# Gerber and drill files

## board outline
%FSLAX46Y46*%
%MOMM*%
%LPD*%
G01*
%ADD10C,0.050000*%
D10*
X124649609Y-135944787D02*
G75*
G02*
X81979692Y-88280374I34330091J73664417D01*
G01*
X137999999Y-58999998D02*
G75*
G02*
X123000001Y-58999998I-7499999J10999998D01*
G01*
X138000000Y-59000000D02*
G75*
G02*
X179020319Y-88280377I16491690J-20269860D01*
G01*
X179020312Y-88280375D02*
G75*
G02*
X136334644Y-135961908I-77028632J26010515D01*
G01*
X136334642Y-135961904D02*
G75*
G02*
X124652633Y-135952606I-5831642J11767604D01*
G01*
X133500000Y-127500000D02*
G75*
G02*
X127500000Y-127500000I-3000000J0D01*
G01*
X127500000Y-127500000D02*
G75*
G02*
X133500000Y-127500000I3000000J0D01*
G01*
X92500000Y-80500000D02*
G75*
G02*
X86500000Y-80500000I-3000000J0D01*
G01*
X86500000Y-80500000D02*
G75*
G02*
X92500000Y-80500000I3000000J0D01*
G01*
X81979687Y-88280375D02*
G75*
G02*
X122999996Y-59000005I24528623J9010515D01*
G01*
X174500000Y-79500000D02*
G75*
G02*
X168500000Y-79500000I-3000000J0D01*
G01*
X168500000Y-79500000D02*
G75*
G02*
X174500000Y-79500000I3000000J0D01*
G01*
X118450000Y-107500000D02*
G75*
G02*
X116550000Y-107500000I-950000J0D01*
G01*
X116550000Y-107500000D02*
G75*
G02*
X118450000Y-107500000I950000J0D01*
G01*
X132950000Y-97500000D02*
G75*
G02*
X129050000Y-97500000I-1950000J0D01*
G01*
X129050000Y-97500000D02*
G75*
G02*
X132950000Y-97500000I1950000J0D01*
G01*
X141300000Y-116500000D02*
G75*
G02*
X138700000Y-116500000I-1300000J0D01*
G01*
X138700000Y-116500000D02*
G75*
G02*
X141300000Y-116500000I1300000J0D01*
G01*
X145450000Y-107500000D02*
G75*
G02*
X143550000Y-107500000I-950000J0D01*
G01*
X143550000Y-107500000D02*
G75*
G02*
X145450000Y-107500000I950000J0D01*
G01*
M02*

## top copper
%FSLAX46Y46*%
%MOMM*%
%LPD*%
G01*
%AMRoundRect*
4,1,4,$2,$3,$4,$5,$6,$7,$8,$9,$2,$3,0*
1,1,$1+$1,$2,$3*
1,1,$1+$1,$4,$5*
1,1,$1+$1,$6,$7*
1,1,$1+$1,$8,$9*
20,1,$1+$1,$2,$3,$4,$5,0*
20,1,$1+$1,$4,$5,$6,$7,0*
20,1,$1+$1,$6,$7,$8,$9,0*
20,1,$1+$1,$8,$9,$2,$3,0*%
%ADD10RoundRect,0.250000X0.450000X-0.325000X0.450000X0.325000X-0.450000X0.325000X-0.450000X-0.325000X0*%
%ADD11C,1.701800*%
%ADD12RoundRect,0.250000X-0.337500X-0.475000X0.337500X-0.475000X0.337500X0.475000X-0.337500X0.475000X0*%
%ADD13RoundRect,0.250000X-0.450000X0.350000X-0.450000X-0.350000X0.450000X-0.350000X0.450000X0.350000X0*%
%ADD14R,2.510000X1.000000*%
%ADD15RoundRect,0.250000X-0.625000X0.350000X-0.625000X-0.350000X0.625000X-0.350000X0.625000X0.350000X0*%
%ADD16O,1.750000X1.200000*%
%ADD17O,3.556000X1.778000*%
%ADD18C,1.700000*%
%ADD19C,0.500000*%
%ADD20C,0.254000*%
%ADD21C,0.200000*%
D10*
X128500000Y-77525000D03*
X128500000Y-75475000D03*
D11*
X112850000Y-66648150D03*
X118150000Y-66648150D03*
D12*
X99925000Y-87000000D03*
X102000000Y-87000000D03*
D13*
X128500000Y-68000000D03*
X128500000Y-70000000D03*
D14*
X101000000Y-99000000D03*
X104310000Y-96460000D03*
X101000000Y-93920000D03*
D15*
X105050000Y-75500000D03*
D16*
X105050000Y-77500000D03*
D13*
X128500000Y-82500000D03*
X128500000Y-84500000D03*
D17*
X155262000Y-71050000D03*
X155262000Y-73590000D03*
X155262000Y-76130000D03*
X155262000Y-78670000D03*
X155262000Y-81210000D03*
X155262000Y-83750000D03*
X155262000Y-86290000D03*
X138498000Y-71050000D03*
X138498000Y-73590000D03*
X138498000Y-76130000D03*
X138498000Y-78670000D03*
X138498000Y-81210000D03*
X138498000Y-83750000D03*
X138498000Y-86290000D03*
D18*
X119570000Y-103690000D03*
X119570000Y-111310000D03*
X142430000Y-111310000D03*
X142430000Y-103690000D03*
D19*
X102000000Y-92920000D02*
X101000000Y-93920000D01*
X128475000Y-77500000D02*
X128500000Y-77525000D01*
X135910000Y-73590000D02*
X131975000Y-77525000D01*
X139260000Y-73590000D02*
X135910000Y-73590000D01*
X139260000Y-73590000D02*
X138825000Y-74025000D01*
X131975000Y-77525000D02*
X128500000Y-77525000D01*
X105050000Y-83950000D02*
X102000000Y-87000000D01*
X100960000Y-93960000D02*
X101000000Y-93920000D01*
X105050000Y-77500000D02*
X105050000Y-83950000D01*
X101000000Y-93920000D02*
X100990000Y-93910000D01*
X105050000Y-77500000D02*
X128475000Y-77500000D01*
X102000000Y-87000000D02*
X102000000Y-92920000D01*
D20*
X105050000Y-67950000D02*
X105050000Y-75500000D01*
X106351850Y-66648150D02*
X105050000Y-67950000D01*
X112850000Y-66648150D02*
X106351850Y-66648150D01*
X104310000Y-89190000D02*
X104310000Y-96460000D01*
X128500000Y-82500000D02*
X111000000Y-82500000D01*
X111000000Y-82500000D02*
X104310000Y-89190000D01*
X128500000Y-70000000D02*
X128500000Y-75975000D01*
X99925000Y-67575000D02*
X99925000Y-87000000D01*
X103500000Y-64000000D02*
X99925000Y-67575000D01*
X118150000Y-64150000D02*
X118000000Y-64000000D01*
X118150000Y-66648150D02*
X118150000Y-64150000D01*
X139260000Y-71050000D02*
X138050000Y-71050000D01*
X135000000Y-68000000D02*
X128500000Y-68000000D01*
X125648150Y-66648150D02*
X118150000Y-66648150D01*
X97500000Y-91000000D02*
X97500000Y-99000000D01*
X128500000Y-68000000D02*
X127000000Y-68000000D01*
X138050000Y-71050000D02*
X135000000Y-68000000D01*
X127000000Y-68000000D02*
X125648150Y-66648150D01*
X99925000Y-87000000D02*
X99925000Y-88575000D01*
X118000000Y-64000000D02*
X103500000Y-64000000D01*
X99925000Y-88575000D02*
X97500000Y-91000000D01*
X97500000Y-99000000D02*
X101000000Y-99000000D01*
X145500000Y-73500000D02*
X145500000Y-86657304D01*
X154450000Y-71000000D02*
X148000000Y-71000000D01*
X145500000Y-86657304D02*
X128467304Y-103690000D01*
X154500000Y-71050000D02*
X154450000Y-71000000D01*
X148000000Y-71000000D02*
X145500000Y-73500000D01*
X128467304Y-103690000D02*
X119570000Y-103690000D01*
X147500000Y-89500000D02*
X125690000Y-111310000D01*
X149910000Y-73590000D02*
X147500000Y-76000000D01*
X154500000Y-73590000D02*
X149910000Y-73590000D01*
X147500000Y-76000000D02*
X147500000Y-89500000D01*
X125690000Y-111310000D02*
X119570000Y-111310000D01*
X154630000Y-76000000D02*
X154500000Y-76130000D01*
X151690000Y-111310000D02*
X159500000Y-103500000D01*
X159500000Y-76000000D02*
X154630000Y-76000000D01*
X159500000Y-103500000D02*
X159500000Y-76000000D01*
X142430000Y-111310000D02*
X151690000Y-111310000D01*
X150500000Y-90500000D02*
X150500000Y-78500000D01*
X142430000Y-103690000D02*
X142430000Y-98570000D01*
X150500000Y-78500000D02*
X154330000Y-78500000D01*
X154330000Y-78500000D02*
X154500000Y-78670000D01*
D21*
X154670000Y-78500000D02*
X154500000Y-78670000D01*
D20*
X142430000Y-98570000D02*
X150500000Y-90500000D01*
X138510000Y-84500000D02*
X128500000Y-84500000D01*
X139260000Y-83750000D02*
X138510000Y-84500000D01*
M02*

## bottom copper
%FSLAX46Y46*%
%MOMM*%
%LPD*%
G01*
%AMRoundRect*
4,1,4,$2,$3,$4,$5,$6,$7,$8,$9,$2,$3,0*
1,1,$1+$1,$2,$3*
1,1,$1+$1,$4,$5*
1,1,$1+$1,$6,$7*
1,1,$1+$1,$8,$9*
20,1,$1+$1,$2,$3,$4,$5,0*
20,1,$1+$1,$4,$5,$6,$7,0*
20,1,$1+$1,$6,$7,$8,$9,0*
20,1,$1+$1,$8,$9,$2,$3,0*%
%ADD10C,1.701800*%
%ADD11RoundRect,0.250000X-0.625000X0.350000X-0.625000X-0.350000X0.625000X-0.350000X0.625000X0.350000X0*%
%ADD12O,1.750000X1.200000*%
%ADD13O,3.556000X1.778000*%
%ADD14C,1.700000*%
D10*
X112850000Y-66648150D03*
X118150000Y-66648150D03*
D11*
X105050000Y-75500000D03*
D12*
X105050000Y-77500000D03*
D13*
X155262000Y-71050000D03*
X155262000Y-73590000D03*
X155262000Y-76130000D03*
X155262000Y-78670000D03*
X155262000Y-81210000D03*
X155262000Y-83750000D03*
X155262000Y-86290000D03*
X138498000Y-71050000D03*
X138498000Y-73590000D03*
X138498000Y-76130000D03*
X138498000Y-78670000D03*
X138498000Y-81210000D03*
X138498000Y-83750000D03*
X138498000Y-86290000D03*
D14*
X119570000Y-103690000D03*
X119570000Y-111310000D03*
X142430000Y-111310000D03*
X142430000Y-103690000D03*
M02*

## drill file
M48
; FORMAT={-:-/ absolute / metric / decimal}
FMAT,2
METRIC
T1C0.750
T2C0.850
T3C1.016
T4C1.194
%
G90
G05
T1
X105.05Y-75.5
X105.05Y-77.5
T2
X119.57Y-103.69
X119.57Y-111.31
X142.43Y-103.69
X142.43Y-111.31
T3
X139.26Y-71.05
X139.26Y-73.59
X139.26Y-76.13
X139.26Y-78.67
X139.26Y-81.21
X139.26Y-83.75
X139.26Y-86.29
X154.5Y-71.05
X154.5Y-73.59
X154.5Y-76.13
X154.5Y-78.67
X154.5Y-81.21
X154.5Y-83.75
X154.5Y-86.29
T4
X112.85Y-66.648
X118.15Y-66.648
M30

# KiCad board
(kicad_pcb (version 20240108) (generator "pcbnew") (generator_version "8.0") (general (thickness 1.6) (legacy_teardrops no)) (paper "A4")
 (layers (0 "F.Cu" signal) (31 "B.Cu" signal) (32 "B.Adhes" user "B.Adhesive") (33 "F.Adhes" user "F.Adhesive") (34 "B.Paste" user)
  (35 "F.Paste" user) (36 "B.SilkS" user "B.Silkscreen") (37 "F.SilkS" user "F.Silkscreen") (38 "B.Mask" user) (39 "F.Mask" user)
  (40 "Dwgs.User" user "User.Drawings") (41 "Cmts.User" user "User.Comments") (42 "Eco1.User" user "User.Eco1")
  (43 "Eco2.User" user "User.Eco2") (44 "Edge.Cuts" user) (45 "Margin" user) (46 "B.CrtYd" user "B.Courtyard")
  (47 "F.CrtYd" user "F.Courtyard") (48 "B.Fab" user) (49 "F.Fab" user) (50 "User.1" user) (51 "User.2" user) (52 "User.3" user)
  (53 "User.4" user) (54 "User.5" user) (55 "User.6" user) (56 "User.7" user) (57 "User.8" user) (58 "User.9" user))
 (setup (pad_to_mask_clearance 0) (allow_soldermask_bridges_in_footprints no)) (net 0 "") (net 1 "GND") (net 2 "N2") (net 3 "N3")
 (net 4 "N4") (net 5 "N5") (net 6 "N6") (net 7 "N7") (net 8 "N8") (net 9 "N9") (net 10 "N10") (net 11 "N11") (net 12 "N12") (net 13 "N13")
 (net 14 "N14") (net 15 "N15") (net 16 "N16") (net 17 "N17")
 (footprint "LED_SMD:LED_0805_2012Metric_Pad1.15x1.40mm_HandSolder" (layer "F.Cu") (at 128.5 76.5 90)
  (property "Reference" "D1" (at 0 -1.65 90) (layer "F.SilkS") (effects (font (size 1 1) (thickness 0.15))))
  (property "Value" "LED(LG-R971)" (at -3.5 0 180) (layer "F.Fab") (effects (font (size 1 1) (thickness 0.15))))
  (pad "1" smd roundrect (at -1.025 0 90) (size 1.15 1.4) (layers "F.Cu" "F.Paste" "F.Mask") (roundrect_rratio 0.217391) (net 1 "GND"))
  (pad "2" smd roundrect (at 1.025 0 90) (size 1.15 1.4) (layers "F.Cu" "F.Paste" "F.Mask") (roundrect_rratio 0.217391) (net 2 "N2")))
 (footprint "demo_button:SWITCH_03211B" (layer "F.Cu") (at 112.85 66.64815 90)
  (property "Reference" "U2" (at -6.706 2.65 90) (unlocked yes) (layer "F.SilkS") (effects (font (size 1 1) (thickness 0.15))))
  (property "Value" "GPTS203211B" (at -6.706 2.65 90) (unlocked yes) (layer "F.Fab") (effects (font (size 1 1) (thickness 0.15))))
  (pad "1" thru_hole circle (at 0 0 90) (size 1.7018 1.7018) (drill 1.1938) (layers "*.Cu" "*.Mask") (remove_unused_layers no) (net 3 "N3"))
  (pad "6" thru_hole circle (at 0 5.3 90) (size 1.7018 1.7018) (drill 1.1938) (layers "*.Cu" "*.Mask") (remove_unused_layers no)
   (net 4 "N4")))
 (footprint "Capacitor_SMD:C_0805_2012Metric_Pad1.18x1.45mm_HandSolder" (layer "F.Cu") (at 100.9625 87)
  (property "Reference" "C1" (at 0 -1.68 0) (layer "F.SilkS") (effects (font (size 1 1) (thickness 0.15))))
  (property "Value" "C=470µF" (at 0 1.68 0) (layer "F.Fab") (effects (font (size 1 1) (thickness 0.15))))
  (pad "1" smd roundrect (at -1.0375 0) (size 1.175 1.45) (layers "F.Cu" "F.Paste" "F.Mask") (roundrect_rratio 0.212766) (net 4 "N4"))
  (pad "2" smd roundrect (at 1.0375 0) (size 1.175 1.45) (layers "F.Cu" "F.Paste" "F.Mask") (roundrect_rratio 0.212766) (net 1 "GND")))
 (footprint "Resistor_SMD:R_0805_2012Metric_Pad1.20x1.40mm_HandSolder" (layer "F.Cu") (at 128.5 69 -90)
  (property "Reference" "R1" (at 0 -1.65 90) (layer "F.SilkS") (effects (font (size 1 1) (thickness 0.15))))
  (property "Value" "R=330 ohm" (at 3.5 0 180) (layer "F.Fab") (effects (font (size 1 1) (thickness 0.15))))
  (pad "1" smd roundrect (at -1 0 270) (size 1.2 1.4) (layers "F.Cu" "F.Paste" "F.Mask") (roundrect_rratio 0.208333) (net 4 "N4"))
  (pad "2" smd roundrect (at 1 0 270) (size 1.2 1.4) (layers "F.Cu" "F.Paste" "F.Mask") (roundrect_rratio 0.208333) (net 2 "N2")))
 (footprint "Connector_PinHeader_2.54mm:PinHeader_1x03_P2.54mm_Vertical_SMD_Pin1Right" (layer "F.Cu") (at 102.655 96.46 180)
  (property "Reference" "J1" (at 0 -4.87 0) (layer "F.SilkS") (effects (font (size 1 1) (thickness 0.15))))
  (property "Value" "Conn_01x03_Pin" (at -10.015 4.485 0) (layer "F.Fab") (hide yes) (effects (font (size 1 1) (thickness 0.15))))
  (pad "1" smd rect (at 1.655 -2.54 180) (size 2.51 1) (layers "F.Cu" "F.Paste" "F.Mask") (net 4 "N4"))
  (pad "2" smd rect (at -1.655 0 180) (size 2.51 1) (layers "F.Cu" "F.Paste" "F.Mask") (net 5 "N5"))
  (pad "3" smd rect (at 1.655 2.54 180) (size 2.51 1) (layers "F.Cu" "F.Paste" "F.Mask") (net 1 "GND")))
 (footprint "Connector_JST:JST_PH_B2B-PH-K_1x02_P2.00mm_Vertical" (layer "F.Cu") (at 105.05 75.5 -90)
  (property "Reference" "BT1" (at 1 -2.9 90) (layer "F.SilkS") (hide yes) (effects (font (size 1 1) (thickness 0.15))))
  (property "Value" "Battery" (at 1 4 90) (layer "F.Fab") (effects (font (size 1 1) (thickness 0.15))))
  (pad "1" thru_hole roundrect (at 0 0 270) (size 1.2 1.75) (drill 0.75) (layers "*.Cu" "*.Mask") (remove_unused_layers no)
   (roundrect_rratio 0.208333) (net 3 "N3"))
  (pad "2" thru_hole oval (at 2 0 270) (size 1.2 1.75) (drill 0.75) (layers "*.Cu" "*.Mask") (remove_unused_layers no) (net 1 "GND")))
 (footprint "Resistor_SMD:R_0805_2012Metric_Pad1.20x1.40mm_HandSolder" (layer "F.Cu") (at 128.5 83.5 -90)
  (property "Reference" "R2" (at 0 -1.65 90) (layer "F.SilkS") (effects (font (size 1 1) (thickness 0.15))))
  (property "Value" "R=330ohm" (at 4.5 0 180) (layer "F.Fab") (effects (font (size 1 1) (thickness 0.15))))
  (pad "1" smd roundrect (at -1 0 270) (size 1.2 1.4) (layers "F.Cu" "F.Paste" "F.Mask") (roundrect_rratio 0.208333) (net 5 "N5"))
  (pad "2" smd roundrect (at 1 0 270) (size 1.2 1.4) (layers "F.Cu" "F.Paste" "F.Mask") (roundrect_rratio 0.208333) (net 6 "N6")))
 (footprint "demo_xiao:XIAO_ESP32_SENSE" (layer "B.Cu") (at 146.88 78.67 180)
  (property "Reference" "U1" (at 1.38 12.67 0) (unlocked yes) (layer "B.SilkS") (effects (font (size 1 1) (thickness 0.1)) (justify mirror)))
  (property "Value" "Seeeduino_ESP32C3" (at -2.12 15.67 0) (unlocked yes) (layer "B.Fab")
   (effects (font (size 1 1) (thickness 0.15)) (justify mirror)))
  (pad "1" thru_hole oval (at -7.62 7.62 180) (size 3.556 1.778) (drill 1.016 (offset -0.762 0)) (layers "*.Cu" "*.Mask")
   (remove_unused_layers no) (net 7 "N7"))
  (pad "2" thru_hole oval (at -7.62 5.08 180) (size 3.556 1.778) (drill 1.016 (offset -0.762 0)) (layers "*.Cu" "*.Mask")
   (remove_unused_layers no) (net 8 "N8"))
  (pad "3" thru_hole oval (at -7.62 2.54 180) (size 3.556 1.778) (drill 1.016 (offset -0.762 0)) (layers "*.Cu" "*.Mask")
   (remove_unused_layers no) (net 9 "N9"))
  (pad "4" thru_hole oval (at -7.62 0 180) (size 3.556 1.778) (drill 1.016 (offset -0.762 0)) (layers "*.Cu" "*.Mask")
   (remove_unused_layers no) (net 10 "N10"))
  (pad "5" thru_hole oval (at -7.62 -2.54 180) (size 3.556 1.778) (drill 1.016 (offset -0.762 0)) (layers "*.Cu" "*.Mask")
   (remove_unused_layers no) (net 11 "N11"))
  (pad "6" thru_hole oval (at -7.62 -5.08 180) (size 3.556 1.778) (drill 1.016 (offset -0.762 0)) (layers "*.Cu" "*.Mask")
   (remove_unused_layers no) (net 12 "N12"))
  (pad "7" thru_hole oval (at -7.62 -7.62 180) (size 3.556 1.778) (drill 1.016 (offset -0.762 0)) (layers "*.Cu" "*.Mask")
   (remove_unused_layers no) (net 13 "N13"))
  (pad "8" thru_hole oval (at 7.62 7.62 180) (size 3.556 1.778) (drill 1.016 (offset 0.762 0)) (layers "*.Cu" "*.Mask")
   (remove_unused_layers no) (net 4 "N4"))
  (pad "9" thru_hole oval (at 7.62 5.08 180) (size 3.556 1.778) (drill 1.016 (offset 0.762 0)) (layers "*.Cu" "*.Mask")
   (remove_unused_layers no) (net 1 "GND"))
  (pad "10" thru_hole oval (at 7.62 2.54 180) (size 3.556 1.778) (drill 1.016 (offset 0.762 0)) (layers "*.Cu" "*.Mask")
   (remove_unused_layers no) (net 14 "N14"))
  (pad "11" thru_hole oval (at 7.62 0 180) (size 3.556 1.778) (drill 1.016 (offset 0.762 0)) (layers "*.Cu" "*.Mask")
   (remove_unused_layers no) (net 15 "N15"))
  (pad "12" thru_hole oval (at 7.62 -2.54 180) (size 3.556 1.778) (drill 1.016 (offset 0.762 0)) (layers "*.Cu" "*.Mask")
   (remove_unused_layers no) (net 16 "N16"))
  (pad "13" thru_hole oval (at 7.62 -5.08 180) (size 3.556 1.778) (drill 1.016 (offset 0.762 0)) (layers "*.Cu" "*.Mask")
   (remove_unused_layers no) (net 6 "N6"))
  (pad "14" thru_hole oval (at 7.62 -7.62 180) (size 3.556 1.778) (drill 1.016 (offset 0.762 0)) (layers "*.Cu" "*.Mask")
   (remove_unused_layers no) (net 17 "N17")))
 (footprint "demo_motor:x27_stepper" (layer "B.Cu") (at 128.46 117.66 180)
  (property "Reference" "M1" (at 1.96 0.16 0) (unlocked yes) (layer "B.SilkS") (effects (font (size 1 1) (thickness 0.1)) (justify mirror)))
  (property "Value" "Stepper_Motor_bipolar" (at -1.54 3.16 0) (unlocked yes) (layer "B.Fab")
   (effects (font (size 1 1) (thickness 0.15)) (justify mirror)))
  (fp_circle (center 10.96 10.16) (end 11.91 10.16) (stroke (width 0.05) (type default)) (fill none) (layer "Edge.Cuts"))
  (fp_circle (center -2.54 20.16) (end -0.59 20.16) (stroke (width 0.05) (type default)) (fill none) (layer "Edge.Cuts"))
  (fp_circle (center -11.54 1.16) (end -10.24 1.16) (stroke (width 0.05) (type default)) (fill none) (layer "Edge.Cuts"))
  (fp_circle (center -16.04 10.16) (end -15.09 10.16) (stroke (width 0.05) (type default)) (fill none) (layer "Edge.Cuts"))
  (pad "1" thru_hole circle (at 8.89 13.97 180) (size 1.7 1.7) (drill 0.85) (layers "*.Cu" "*.Mask") (remove_unused_layers no) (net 7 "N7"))
  (pad "2" thru_hole circle (at 8.89 6.35 180) (size 1.7 1.7) (drill 0.85) (layers "*.Cu" "*.Mask") (remove_unused_layers no) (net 8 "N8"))
  (pad "3" thru_hole circle (at -13.97 6.35 180) (size 1.7 1.7) (drill 0.85) (layers "*.Cu" "*.Mask") (remove_unused_layers no) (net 9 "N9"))
  (pad "4" thru_hole circle (at -13.97 13.97 180) (size 1.7 1.7) (drill 0.85) (layers "*.Cu" "*.Mask") (remove_unused_layers no)
   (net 10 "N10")))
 (gr_arc (start 124.649609 135.944787) (mid 98.427474 116.487655) (end 81.979688 88.280375) (stroke (width 0.05) (type default))
  (layer "Edge.Cuts"))
 (gr_arc (start 137.999999 58.999998) (mid 130.5 61.313525) (end 123.000001 58.999999) (stroke (width 0.05) (type default))
  (layer "Edge.Cuts"))
 (gr_arc (start 138 59) (mid 169.67336 58.001109) (end 179.020313 88.280375) (stroke (width 0.05) (type default)) (layer "Edge.Cuts"))
 (gr_arc (start 179.020312 88.280375) (mid 162.566345 116.497774) (end 136.334642 135.961904) (stroke (width 0.05) (type default))
  (layer "Edge.Cuts"))
 (gr_arc (start 136.334642 135.961904) (mid 130.492551 137.327611) (end 124.65265 135.952573) (stroke (width 0.05) (type default))
  (layer "Edge.Cuts"))
 (gr_circle (center 130.5 127.5) (end 133.5 127.5) (stroke (width 0.05) (type default)) (fill none) (layer "Edge.Cuts"))
 (gr_circle (center 89.5 80.5) (end 92.5 80.5) (stroke (width 0.05) (type default)) (fill none) (layer "Edge.Cuts"))
 (gr_arc (start 81.979687 88.280375) (mid 91.32664 58.001109) (end 123 59) (stroke (width 0.05) (type default)) (layer "Edge.Cuts"))
 (gr_circle (center 171.5 79.5) (end 174.5 79.5) (stroke (width 0.05) (type default)) (fill none) (layer "Edge.Cuts"))
 (segment (start 102 92.92) (end 101 93.92) (width 0.5) (layer "F.Cu") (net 1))
 (segment (start 128.475 77.5) (end 128.5 77.525) (width 0.5) (layer "F.Cu") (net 1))
 (segment (start 135.91 73.59) (end 131.975 77.525) (width 0.5) (layer "F.Cu") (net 1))
 (segment (start 139.26 73.59) (end 135.91 73.59) (width 0.5) (layer "F.Cu") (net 1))
 (segment (start 139.26 73.59) (end 138.825 74.025) (width 0.5) (layer "F.Cu") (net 1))
 (segment (start 131.975 77.525) (end 128.5 77.525) (width 0.5) (layer "F.Cu") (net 1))
 (segment (start 105.05 83.95) (end 102 87) (width 0.5) (layer "F.Cu") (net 1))
 (segment (start 100.96 93.96) (end 101 93.92) (width 0.5) (layer "F.Cu") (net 1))
 (segment (start 105.05 77.5) (end 105.05 83.95) (width 0.5) (layer "F.Cu") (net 1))
 (segment (start 101 93.92) (end 100.99 93.91) (width 0.5) (layer "F.Cu") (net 1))
 (segment (start 105.05 77.5) (end 128.475 77.5) (width 0.5) (layer "F.Cu") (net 1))
 (segment (start 102 87) (end 102 92.92) (width 0.5) (layer "F.Cu") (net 1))
 (segment (start 105.05 67.95) (end 105.05 75.5) (width 0.254) (layer "F.Cu") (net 3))
 (segment (start 106.35185 66.64815) (end 105.05 67.95) (width 0.254) (layer "F.Cu") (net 3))
 (segment (start 112.85 66.64815) (end 106.35185 66.64815) (width 0.254) (layer "F.Cu") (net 3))
 (segment (start 104.31 89.19) (end 104.31 96.46) (width 0.254) (layer "F.Cu") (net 5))
 (segment (start 128.5 82.5) (end 111 82.5) (width 0.254) (layer "F.Cu") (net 5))
 (segment (start 111 82.5) (end 104.31 89.19) (width 0.254) (layer "F.Cu") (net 5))
 (segment (start 128.5 70) (end 128.5 75.975) (width 0.254) (layer "F.Cu") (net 2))
 (segment (start 99.925 67.575) (end 99.925 87) (width 0.254) (layer "F.Cu") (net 4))
 (segment (start 103.5 64) (end 99.925 67.575) (width 0.254) (layer "F.Cu") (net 4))
 (segment (start 118.15 64.15) (end 118 64) (width 0.254) (layer "F.Cu") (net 4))
 (segment (start 118.15 66.64815) (end 118.15 64.15) (width 0.254) (layer "F.Cu") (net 4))
 (segment (start 139.26 71.05) (end 138.05 71.05) (width 0.254) (layer "F.Cu") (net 4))
 (segment (start 135 68) (end 128.5 68) (width 0.254) (layer "F.Cu") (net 4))
 (segment (start 125.64815 66.64815) (end 118.15 66.64815) (width 0.254) (layer "F.Cu") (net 4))
 (segment (start 97.5 91) (end 97.5 99) (width 0.254) (layer "F.Cu") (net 4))
 (segment (start 128.5 68) (end 127 68) (width 0.254) (layer "F.Cu") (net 4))
 (segment (start 138.05 71.05) (end 135 68) (width 0.254) (layer "F.Cu") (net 4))
 (segment (start 127 68) (end 125.64815 66.64815) (width 0.254) (layer "F.Cu") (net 4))
 (segment (start 99.925 87) (end 99.925 88.575) (width 0.254) (layer "F.Cu") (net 4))
 (segment (start 118 64) (end 103.5 64) (width 0.254) (layer "F.Cu") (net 4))
 (segment (start 99.925 88.575) (end 97.5 91) (width 0.254) (layer "F.Cu") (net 4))
 (segment (start 97.5 99) (end 101 99) (width 0.254) (layer "F.Cu") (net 4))
 (segment (start 145.5 73.5) (end 145.5 86.657304) (width 0.254) (layer "F.Cu") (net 7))
 (segment (start 154.45 71) (end 148 71) (width 0.254) (layer "F.Cu") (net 7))
 (segment (start 145.5 86.657304) (end 128.467304 103.69) (width 0.254) (layer "F.Cu") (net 7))
 (segment (start 154.5 71.05) (end 154.45 71) (width 0.254) (layer "F.Cu") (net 7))
 (segment (start 148 71) (end 145.5 73.5) (width 0.254) (layer "F.Cu") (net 7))
 (segment (start 128.467304 103.69) (end 119.57 103.69) (width 0.254) (layer "F.Cu") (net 7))
 (segment (start 147.5 89.5) (end 125.69 111.31) (width 0.254) (layer "F.Cu") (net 8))
 (segment (start 149.91 73.59) (end 147.5 76) (width 0.254) (layer "F.Cu") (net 8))
 (segment (start 154.5 73.59) (end 149.91 73.59) (width 0.254) (layer "F.Cu") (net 8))
 (segment (start 147.5 76) (end 147.5 89.5) (width 0.254) (layer "F.Cu") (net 8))
 (segment (start 125.69 111.31) (end 119.57 111.31) (width 0.254) (layer "F.Cu") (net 8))
 (segment (start 154.63 76) (end 154.5 76.13) (width 0.254) (layer "F.Cu") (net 9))
 (segment (start 151.69 111.31) (end 159.5 103.5) (width 0.254) (layer "F.Cu") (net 9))
 (segment (start 159.5 76) (end 154.63 76) (width 0.254) (layer "F.Cu") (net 9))
 (segment (start 159.5 103.5) (end 159.5 76) (width 0.254) (layer "F.Cu") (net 9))
 (segment (start 142.43 111.31) (end 151.69 111.31) (width 0.254) (layer "F.Cu") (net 9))
 (segment (start 150.5 90.5) (end 150.5 78.5) (width 0.254) (layer "F.Cu") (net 10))
 (segment (start 142.43 103.69) (end 142.43 98.57) (width 0.254) (layer "F.Cu") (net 10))
 (segment (start 150.5 78.5) (end 154.33 78.5) (width 0.254) (layer "F.Cu") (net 10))
 (segment (start 154.33 78.5) (end 154.5 78.67) (width 0.254) (layer "F.Cu") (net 10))
 (segment (start 154.67 78.5) (end 154.5 78.67) (width 0.2) (layer "F.Cu") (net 10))
 (segment (start 142.43 98.57) (end 150.5 90.5) (width 0.254) (layer "F.Cu") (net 10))
 (segment (start 138.51 84.5) (end 128.5 84.5) (width 0.254) (layer "F.Cu") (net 6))
 (segment (start 139.26 83.75) (end 138.51 84.5) (width 0.254) (layer "F.Cu") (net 6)))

